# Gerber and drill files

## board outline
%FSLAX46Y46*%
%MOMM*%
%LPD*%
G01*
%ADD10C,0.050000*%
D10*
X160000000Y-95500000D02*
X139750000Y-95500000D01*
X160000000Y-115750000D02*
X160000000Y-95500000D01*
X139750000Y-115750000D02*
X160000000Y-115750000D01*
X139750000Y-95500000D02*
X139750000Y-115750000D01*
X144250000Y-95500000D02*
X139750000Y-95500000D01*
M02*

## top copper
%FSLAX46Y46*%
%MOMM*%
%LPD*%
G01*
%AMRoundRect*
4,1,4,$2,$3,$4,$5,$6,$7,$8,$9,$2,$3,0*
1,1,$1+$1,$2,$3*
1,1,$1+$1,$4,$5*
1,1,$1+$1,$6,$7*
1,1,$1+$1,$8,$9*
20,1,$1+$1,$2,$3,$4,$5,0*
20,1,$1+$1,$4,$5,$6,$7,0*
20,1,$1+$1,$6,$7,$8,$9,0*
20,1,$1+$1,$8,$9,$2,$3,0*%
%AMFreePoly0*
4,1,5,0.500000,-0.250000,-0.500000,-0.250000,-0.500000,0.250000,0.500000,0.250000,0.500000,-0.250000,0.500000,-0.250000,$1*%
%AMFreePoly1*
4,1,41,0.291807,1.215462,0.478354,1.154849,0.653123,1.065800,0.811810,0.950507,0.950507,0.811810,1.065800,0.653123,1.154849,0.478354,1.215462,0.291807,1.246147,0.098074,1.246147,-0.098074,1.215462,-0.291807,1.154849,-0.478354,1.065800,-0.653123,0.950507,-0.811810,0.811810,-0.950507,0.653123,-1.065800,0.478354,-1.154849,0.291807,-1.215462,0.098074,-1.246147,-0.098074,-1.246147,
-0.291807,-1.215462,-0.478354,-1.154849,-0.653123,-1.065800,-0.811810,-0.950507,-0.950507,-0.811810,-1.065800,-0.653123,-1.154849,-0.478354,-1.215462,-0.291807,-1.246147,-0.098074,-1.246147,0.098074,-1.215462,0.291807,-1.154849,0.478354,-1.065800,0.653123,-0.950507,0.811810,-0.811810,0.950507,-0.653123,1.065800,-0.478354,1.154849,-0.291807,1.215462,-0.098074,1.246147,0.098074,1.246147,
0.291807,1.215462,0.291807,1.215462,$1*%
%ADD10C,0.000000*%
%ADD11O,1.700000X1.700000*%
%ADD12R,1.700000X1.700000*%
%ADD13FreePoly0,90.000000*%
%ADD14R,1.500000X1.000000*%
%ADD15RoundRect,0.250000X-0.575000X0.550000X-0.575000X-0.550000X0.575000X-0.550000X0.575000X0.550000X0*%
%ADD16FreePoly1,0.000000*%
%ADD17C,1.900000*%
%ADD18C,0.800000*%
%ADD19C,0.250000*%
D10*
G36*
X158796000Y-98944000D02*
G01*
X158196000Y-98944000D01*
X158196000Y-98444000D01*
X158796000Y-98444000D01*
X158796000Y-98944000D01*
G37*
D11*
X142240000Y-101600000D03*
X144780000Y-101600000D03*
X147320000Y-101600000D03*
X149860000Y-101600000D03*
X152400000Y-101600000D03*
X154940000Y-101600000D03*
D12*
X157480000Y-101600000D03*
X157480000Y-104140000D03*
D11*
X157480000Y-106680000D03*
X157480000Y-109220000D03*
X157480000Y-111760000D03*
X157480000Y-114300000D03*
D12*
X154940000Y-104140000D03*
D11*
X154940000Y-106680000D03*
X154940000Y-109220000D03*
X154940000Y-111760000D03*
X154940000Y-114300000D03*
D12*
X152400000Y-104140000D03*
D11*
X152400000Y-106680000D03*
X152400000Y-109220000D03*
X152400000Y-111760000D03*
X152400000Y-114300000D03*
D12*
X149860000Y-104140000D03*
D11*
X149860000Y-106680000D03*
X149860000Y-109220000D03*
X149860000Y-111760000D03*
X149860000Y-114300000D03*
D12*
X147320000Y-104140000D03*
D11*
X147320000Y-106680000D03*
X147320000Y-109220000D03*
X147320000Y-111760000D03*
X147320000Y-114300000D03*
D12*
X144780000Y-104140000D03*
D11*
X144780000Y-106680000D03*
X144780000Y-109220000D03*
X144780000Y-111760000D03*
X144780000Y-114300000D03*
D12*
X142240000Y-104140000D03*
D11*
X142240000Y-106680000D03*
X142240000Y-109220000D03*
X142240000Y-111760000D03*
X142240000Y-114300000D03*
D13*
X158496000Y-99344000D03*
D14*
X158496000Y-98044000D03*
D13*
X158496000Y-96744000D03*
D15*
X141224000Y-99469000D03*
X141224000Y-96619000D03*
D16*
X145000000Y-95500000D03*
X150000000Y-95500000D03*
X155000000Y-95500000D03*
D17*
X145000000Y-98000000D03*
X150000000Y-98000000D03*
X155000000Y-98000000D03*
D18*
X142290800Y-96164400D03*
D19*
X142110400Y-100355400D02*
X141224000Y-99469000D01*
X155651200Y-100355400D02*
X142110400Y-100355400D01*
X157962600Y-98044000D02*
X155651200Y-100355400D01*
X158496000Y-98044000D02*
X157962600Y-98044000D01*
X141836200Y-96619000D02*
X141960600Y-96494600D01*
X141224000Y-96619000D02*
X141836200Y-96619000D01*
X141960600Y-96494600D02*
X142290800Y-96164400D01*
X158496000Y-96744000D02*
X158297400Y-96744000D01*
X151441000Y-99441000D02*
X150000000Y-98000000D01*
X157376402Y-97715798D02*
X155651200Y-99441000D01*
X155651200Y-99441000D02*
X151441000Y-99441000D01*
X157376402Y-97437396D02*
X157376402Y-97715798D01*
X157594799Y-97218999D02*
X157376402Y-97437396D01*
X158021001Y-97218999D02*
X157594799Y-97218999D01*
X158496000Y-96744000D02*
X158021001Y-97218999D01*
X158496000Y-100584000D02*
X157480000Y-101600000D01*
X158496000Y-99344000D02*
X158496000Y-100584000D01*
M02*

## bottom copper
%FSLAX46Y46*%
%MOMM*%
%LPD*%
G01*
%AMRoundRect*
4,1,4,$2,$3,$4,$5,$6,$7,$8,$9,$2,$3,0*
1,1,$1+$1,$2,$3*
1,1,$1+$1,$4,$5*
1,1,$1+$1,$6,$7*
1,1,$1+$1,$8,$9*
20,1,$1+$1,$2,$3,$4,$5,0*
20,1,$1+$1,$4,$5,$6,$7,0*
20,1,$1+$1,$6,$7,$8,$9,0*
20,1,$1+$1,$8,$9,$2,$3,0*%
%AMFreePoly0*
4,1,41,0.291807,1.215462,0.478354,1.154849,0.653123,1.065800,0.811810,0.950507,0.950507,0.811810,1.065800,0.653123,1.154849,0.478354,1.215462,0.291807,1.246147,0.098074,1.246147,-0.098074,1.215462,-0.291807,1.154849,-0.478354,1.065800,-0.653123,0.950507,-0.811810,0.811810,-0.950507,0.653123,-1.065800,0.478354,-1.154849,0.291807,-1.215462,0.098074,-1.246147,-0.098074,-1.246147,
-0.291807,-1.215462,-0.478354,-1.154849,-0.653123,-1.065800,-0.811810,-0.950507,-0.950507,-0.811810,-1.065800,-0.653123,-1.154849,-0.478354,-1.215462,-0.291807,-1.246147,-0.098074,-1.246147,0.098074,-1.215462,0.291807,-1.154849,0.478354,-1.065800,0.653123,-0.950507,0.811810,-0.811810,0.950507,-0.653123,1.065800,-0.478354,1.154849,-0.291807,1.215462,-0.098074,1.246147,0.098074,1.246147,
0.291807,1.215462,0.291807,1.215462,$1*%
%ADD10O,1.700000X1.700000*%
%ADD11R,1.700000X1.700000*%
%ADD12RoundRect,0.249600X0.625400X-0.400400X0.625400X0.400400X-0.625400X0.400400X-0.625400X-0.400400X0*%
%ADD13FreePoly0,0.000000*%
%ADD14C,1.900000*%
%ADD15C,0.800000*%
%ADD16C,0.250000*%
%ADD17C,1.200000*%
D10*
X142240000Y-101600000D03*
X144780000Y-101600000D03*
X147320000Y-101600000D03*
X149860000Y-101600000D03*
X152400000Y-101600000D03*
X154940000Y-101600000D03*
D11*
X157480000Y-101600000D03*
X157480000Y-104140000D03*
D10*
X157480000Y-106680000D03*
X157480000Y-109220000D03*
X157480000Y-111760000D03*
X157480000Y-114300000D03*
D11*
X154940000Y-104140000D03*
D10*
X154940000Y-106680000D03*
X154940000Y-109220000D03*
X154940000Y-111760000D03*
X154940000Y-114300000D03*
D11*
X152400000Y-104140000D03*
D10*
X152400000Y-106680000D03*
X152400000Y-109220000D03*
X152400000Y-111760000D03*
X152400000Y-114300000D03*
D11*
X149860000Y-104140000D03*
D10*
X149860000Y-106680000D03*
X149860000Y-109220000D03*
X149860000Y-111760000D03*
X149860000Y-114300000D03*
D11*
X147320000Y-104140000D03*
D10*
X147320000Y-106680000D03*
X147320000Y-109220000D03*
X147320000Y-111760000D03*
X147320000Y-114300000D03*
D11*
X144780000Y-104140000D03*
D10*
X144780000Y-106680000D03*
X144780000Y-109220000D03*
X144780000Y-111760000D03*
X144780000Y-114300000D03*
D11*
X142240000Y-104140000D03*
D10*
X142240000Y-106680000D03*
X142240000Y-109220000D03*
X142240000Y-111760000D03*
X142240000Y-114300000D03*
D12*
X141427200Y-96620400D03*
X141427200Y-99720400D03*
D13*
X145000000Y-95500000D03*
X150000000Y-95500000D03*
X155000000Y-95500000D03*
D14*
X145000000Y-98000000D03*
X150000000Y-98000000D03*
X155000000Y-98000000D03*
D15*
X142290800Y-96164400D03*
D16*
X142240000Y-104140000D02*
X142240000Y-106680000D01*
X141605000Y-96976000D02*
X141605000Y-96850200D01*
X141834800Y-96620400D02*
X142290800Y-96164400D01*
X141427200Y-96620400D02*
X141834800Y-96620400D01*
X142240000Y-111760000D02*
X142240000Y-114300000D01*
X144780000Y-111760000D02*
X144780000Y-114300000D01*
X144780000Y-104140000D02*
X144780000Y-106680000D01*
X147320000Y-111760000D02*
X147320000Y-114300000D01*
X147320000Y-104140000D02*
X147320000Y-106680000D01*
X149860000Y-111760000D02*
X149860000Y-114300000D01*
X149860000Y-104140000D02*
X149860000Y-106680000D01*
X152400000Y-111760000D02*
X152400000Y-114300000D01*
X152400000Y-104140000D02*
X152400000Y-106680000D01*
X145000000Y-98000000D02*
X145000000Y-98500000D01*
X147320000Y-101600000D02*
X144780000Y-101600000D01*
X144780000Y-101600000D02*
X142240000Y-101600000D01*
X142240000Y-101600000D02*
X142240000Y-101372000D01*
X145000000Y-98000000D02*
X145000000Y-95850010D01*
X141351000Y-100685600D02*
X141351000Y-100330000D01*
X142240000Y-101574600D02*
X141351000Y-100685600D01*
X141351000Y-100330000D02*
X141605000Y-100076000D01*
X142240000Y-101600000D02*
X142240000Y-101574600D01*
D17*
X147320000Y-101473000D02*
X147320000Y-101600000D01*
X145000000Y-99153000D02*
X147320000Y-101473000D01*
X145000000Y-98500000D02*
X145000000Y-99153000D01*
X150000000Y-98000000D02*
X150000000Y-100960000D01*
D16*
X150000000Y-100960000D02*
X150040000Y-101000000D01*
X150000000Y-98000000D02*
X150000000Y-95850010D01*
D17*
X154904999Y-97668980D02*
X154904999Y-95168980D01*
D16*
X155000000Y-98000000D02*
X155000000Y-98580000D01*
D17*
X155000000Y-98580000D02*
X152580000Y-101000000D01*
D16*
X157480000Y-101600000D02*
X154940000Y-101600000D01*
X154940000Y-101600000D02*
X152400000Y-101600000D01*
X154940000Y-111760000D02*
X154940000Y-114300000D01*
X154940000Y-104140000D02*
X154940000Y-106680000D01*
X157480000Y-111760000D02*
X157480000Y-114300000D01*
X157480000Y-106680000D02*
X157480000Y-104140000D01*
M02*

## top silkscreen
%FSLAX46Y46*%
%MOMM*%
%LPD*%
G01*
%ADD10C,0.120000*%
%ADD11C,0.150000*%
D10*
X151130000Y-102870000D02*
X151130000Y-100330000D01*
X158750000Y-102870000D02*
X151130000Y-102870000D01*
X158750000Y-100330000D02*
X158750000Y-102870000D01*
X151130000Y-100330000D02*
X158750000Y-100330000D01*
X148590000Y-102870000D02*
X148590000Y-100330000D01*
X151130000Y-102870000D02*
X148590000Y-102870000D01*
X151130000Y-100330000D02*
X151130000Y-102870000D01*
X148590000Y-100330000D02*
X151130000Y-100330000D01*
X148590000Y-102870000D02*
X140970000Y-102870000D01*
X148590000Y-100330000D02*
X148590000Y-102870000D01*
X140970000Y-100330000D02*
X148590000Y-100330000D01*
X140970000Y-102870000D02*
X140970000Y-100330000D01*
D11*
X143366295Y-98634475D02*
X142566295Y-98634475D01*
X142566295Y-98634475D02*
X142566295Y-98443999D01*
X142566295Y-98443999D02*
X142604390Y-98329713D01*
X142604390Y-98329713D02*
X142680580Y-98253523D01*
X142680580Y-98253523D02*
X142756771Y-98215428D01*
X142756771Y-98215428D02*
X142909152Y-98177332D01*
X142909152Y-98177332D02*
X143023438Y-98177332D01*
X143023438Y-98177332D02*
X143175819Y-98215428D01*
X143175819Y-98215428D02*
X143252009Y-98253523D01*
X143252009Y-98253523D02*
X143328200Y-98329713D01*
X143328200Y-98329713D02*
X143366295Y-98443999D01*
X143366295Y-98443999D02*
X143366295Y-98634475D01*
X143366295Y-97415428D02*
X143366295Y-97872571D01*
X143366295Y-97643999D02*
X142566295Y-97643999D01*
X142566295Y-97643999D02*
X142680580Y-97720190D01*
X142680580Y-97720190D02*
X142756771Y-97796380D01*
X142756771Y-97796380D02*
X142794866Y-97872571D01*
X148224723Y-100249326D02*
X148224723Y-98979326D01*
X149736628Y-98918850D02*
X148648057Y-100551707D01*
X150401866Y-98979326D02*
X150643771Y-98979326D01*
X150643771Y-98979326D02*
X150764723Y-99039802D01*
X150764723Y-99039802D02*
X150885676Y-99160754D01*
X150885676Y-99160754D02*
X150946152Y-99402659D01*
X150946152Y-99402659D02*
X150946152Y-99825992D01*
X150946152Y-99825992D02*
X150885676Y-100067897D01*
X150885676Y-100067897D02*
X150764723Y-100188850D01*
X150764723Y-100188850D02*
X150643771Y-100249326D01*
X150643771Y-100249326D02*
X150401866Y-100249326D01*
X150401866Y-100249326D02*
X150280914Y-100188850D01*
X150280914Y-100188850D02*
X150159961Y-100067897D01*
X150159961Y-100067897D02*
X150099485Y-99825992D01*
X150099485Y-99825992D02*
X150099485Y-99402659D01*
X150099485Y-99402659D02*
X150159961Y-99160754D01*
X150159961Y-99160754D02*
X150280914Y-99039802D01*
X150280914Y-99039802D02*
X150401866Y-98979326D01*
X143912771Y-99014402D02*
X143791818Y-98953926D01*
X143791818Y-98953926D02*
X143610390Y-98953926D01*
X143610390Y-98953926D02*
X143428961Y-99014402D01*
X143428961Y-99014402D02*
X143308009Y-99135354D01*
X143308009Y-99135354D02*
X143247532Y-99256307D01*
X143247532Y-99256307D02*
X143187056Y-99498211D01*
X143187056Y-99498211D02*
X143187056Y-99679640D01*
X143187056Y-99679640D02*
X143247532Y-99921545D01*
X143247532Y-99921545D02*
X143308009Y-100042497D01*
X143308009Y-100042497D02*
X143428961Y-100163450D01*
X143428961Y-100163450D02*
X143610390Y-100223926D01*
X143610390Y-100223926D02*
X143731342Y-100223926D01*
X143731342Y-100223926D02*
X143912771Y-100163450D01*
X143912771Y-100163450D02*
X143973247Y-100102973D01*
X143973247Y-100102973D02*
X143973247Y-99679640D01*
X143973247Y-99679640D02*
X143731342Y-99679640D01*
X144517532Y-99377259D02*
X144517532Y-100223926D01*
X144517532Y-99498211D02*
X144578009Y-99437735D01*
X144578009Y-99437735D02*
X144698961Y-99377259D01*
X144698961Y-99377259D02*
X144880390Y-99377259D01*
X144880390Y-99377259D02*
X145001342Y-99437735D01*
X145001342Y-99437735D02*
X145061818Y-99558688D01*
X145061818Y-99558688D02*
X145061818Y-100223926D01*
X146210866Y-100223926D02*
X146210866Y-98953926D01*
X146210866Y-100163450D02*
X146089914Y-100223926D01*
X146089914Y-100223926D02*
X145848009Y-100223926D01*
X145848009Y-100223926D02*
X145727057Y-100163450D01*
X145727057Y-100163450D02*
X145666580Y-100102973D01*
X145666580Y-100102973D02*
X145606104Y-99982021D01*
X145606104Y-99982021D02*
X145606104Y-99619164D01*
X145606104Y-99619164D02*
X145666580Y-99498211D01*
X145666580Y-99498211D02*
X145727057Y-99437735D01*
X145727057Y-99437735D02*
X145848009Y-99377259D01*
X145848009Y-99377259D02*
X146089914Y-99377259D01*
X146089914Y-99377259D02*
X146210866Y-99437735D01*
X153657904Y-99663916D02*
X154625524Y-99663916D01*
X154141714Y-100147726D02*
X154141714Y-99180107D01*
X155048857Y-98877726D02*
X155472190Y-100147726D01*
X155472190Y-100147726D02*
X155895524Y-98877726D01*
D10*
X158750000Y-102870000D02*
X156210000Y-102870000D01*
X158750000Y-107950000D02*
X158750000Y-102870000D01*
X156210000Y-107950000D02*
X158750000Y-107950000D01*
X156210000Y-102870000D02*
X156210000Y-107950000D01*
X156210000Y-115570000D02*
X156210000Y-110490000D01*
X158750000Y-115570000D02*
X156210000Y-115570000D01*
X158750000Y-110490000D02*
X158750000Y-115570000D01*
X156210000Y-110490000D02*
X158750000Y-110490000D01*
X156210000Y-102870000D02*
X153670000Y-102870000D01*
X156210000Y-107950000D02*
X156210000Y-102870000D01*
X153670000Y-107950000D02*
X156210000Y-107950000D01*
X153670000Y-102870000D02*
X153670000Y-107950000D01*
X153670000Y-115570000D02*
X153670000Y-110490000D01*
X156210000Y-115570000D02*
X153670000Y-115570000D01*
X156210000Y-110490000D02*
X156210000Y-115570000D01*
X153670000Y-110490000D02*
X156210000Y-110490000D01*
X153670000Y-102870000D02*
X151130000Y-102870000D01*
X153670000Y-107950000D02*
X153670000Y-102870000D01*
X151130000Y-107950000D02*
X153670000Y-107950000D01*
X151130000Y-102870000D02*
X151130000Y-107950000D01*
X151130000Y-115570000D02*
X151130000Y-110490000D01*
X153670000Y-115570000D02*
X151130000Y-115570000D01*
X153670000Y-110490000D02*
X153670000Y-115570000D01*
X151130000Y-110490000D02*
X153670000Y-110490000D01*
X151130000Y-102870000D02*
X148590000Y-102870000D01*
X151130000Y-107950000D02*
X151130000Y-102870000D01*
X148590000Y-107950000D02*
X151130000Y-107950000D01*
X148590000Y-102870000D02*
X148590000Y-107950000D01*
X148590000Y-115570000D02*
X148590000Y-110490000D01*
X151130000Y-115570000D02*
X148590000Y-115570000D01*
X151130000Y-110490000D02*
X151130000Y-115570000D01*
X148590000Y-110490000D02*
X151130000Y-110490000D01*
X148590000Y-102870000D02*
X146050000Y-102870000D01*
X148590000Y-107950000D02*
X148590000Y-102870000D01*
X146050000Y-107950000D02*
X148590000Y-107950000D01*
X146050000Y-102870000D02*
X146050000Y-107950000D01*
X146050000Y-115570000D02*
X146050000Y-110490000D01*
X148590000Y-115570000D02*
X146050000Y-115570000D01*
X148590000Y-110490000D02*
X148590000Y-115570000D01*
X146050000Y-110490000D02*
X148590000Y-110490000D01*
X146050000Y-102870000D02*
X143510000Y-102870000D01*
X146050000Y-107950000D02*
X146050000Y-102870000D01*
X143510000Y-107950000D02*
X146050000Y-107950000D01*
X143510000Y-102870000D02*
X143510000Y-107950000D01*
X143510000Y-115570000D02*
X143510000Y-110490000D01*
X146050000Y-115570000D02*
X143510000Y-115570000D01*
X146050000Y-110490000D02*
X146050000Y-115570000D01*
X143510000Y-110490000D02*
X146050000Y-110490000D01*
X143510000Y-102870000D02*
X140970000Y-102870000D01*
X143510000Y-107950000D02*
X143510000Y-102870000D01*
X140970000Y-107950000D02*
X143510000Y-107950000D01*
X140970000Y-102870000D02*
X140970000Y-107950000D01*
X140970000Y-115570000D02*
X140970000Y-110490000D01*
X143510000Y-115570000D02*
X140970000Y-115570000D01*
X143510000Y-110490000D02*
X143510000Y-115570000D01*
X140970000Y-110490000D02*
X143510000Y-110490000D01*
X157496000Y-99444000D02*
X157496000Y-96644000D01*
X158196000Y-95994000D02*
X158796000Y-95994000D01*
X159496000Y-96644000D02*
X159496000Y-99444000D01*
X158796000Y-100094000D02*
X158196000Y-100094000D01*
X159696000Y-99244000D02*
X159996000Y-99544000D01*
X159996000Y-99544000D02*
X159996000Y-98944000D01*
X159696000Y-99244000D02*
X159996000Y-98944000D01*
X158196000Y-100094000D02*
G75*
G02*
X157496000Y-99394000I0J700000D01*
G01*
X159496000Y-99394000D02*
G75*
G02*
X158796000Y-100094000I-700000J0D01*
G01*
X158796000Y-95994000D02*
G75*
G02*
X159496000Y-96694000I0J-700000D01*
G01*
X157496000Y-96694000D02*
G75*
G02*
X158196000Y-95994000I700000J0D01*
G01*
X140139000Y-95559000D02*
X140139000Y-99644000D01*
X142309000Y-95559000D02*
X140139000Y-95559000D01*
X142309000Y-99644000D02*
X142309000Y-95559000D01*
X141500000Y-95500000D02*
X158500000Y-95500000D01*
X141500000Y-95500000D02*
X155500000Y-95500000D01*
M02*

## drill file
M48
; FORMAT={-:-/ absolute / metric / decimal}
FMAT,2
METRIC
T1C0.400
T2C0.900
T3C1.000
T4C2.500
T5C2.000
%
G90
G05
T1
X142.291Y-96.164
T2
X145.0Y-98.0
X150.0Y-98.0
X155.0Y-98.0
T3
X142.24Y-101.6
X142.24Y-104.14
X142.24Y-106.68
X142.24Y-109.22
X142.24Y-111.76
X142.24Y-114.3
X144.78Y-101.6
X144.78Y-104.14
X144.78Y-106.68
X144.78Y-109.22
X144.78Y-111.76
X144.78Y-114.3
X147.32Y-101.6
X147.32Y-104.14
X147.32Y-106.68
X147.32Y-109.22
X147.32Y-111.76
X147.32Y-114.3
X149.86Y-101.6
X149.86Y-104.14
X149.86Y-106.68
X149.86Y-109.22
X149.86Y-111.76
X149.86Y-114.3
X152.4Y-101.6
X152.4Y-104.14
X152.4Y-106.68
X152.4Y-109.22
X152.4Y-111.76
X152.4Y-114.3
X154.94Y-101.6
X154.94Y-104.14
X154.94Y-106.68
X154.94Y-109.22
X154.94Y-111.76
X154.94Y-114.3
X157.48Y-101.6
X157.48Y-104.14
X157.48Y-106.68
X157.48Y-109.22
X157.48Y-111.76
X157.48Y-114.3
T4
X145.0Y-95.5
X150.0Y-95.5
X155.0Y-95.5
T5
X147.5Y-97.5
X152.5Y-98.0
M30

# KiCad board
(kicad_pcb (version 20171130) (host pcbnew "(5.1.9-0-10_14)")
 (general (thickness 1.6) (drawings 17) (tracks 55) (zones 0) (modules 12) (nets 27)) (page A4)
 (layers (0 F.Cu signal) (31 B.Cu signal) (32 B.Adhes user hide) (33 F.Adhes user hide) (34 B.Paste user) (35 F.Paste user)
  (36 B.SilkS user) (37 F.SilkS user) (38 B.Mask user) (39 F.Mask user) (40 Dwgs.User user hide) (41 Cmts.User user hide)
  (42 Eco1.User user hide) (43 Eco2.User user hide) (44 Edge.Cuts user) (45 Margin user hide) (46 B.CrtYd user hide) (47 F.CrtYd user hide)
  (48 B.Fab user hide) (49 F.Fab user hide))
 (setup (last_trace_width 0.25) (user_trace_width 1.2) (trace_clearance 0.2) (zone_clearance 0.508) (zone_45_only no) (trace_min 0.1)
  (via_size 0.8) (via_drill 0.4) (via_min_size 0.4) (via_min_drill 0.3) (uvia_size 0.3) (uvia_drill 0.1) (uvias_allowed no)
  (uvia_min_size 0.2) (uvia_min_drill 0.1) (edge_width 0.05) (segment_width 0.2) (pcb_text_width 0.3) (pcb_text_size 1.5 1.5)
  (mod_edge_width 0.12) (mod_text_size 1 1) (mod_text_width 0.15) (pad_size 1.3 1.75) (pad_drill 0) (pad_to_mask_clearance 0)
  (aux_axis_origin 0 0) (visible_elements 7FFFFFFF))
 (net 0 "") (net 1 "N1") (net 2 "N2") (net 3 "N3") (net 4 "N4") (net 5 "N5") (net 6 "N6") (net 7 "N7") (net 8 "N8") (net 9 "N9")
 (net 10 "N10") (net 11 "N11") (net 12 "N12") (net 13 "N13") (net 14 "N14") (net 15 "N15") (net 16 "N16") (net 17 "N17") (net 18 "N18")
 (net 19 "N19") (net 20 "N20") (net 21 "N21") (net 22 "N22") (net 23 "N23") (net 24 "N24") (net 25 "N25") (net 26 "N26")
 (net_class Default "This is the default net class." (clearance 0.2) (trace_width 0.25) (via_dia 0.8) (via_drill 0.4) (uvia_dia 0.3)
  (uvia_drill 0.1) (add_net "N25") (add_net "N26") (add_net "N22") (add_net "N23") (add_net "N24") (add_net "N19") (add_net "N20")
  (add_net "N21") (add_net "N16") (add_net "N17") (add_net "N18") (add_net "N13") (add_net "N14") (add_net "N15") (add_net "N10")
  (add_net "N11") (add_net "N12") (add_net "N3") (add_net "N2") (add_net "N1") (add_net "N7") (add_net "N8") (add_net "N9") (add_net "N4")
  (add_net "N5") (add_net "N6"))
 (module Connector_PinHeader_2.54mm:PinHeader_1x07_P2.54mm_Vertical (layer F.Cu) (at 157.48 101.6 270)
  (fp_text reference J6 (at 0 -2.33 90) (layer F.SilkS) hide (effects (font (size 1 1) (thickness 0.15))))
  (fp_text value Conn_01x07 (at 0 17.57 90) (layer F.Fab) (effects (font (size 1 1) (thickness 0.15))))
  (pad 7 thru_hole oval (at 0 15.24 270) (size 1.7 1.7) (drill 1) (layers *.Cu *.Mask) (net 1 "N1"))
  (pad 6 thru_hole oval (at 0 12.7 270) (size 1.7 1.7) (drill 1) (layers *.Cu *.Mask) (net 1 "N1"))
  (pad 5 thru_hole oval (at 0 10.16 270) (size 1.7 1.7) (drill 1) (layers *.Cu *.Mask) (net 1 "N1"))
  (pad 4 thru_hole oval (at 0 7.62 270) (size 1.7 1.7) (drill 1) (layers *.Cu *.Mask) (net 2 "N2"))
  (pad 3 thru_hole oval (at 0 5.08 270) (size 1.7 1.7) (drill 1) (layers *.Cu *.Mask) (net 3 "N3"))
  (pad 2 thru_hole oval (at 0 2.54 270) (size 1.7 1.7) (drill 1) (layers *.Cu *.Mask) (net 3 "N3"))
  (pad 1 thru_hole rect (at 0 0 270) (size 1.7 1.7) (drill 1) (layers *.Cu *.Mask) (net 3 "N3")))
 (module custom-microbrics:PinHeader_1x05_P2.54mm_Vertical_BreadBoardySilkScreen (layer F.Cu) (at 157.48 104.14)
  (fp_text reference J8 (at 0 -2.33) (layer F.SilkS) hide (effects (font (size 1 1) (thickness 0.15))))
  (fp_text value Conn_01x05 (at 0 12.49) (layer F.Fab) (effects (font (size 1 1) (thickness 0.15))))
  (fp_line (start 1.27 -1.27) (end -1.27 -1.27) (layer F.SilkS) (width 0.12))
  (fp_line (start 1.27 3.81) (end 1.27 -1.27) (layer F.SilkS) (width 0.12))
  (fp_line (start -1.27 3.81) (end 1.27 3.81) (layer F.SilkS) (width 0.12))
  (fp_line (start -1.27 -1.27) (end -1.27 3.81) (layer F.SilkS) (width 0.12))
  (fp_line (start -1.27 11.43) (end -1.27 6.35) (layer F.SilkS) (width 0.12))
  (fp_line (start 1.27 11.43) (end -1.27 11.43) (layer F.SilkS) (width 0.12))
  (fp_line (start 1.27 6.35) (end 1.27 11.43) (layer F.SilkS) (width 0.12))
  (fp_line (start -1.27 6.35) (end 1.27 6.35) (layer F.SilkS) (width 0.12))
  (pad 1 thru_hole rect (at 0 0) (size 1.7 1.7) (drill 1) (layers *.Cu *.Mask) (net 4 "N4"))
  (pad 2 thru_hole oval (at 0 2.54) (size 1.7 1.7) (drill 1) (layers *.Cu *.Mask) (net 4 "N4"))
  (pad 3 thru_hole oval (at 0 5.08) (size 1.7 1.7) (drill 1) (layers *.Cu *.Mask) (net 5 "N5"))
  (pad 4 thru_hole oval (at 0 7.62) (size 1.7 1.7) (drill 1) (layers *.Cu *.Mask) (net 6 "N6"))
  (pad 5 thru_hole oval (at 0 10.16) (size 1.7 1.7) (drill 1) (layers *.Cu *.Mask) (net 6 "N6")))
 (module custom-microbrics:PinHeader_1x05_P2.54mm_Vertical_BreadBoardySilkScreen (layer F.Cu) (at 154.94 104.14)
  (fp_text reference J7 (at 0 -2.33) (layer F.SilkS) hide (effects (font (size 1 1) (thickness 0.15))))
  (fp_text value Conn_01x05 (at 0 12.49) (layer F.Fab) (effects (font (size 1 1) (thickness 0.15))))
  (fp_line (start 1.27 -1.27) (end -1.27 -1.27) (layer F.SilkS) (width 0.12))
  (fp_line (start 1.27 3.81) (end 1.27 -1.27) (layer F.SilkS) (width 0.12))
  (fp_line (start -1.27 3.81) (end 1.27 3.81) (layer F.SilkS) (width 0.12))
  (fp_line (start -1.27 -1.27) (end -1.27 3.81) (layer F.SilkS) (width 0.12))
  (fp_line (start -1.27 11.43) (end -1.27 6.35) (layer F.SilkS) (width 0.12))
  (fp_line (start 1.27 11.43) (end -1.27 11.43) (layer F.SilkS) (width 0.12))
  (fp_line (start 1.27 6.35) (end 1.27 11.43) (layer F.SilkS) (width 0.12))
  (fp_line (start -1.27 6.35) (end 1.27 6.35) (layer F.SilkS) (width 0.12))
  (pad 1 thru_hole rect (at 0 0) (size 1.7 1.7) (drill 1) (layers *.Cu *.Mask) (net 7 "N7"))
  (pad 2 thru_hole oval (at 0 2.54) (size 1.7 1.7) (drill 1) (layers *.Cu *.Mask) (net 7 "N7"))
  (pad 3 thru_hole oval (at 0 5.08) (size 1.7 1.7) (drill 1) (layers *.Cu *.Mask) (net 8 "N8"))
  (pad 4 thru_hole oval (at 0 7.62) (size 1.7 1.7) (drill 1) (layers *.Cu *.Mask) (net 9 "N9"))
  (pad 5 thru_hole oval (at 0 10.16) (size 1.7 1.7) (drill 1) (layers *.Cu *.Mask) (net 9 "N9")))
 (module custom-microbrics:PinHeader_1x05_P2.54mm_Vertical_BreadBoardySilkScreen (layer F.Cu) (at 152.4 104.14)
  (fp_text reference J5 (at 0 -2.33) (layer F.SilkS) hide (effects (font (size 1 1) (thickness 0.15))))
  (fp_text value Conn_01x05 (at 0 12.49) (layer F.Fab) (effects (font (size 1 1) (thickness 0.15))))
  (fp_line (start 1.27 -1.27) (end -1.27 -1.27) (layer F.SilkS) (width 0.12))
  (fp_line (start 1.27 3.81) (end 1.27 -1.27) (layer F.SilkS) (width 0.12))
  (fp_line (start -1.27 3.81) (end 1.27 3.81) (layer F.SilkS) (width 0.12))
  (fp_line (start -1.27 -1.27) (end -1.27 3.81) (layer F.SilkS) (width 0.12))
  (fp_line (start -1.27 11.43) (end -1.27 6.35) (layer F.SilkS) (width 0.12))
  (fp_line (start 1.27 11.43) (end -1.27 11.43) (layer F.SilkS) (width 0.12))
  (fp_line (start 1.27 6.35) (end 1.27 11.43) (layer F.SilkS) (width 0.12))
  (fp_line (start -1.27 6.35) (end 1.27 6.35) (layer F.SilkS) (width 0.12))
  (pad 1 thru_hole rect (at 0 0) (size 1.7 1.7) (drill 1) (layers *.Cu *.Mask) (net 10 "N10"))
  (pad 2 thru_hole oval (at 0 2.54) (size 1.7 1.7) (drill 1) (layers *.Cu *.Mask) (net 10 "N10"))
  (pad 3 thru_hole oval (at 0 5.08) (size 1.7 1.7) (drill 1) (layers *.Cu *.Mask) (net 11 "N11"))
  (pad 4 thru_hole oval (at 0 7.62) (size 1.7 1.7) (drill 1) (layers *.Cu *.Mask) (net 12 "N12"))
  (pad 5 thru_hole oval (at 0 10.16) (size 1.7 1.7) (drill 1) (layers *.Cu *.Mask) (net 12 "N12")))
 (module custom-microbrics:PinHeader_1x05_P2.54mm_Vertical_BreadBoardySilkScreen (layer F.Cu) (at 149.86 104.14)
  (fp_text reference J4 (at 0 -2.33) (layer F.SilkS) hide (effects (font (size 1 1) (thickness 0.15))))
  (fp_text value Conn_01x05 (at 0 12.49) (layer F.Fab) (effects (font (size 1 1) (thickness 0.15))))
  (fp_line (start 1.27 -1.27) (end -1.27 -1.27) (layer F.SilkS) (width 0.12))
  (fp_line (start 1.27 3.81) (end 1.27 -1.27) (layer F.SilkS) (width 0.12))
  (fp_line (start -1.27 3.81) (end 1.27 3.81) (layer F.SilkS) (width 0.12))
  (fp_line (start -1.27 -1.27) (end -1.27 3.81) (layer F.SilkS) (width 0.12))
  (fp_line (start -1.27 11.43) (end -1.27 6.35) (layer F.SilkS) (width 0.12))
  (fp_line (start 1.27 11.43) (end -1.27 11.43) (layer F.SilkS) (width 0.12))
  (fp_line (start 1.27 6.35) (end 1.27 11.43) (layer F.SilkS) (width 0.12))
  (fp_line (start -1.27 6.35) (end 1.27 6.35) (layer F.SilkS) (width 0.12))
  (pad 1 thru_hole rect (at 0 0) (size 1.7 1.7) (drill 1) (layers *.Cu *.Mask) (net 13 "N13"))
  (pad 2 thru_hole oval (at 0 2.54) (size 1.7 1.7) (drill 1) (layers *.Cu *.Mask) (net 13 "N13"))
  (pad 3 thru_hole oval (at 0 5.08) (size 1.7 1.7) (drill 1) (layers *.Cu *.Mask) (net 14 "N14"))
  (pad 4 thru_hole oval (at 0 7.62) (size 1.7 1.7) (drill 1) (layers *.Cu *.Mask) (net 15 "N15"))
  (pad 5 thru_hole oval (at 0 10.16) (size 1.7 1.7) (drill 1) (layers *.Cu *.Mask) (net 15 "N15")))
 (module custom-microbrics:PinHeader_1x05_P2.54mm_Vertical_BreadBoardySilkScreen (layer F.Cu) (at 147.32 104.14)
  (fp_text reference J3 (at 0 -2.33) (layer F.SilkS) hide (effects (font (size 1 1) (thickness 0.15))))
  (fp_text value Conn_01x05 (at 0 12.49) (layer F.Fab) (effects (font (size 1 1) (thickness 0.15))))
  (fp_line (start 1.27 -1.27) (end -1.27 -1.27) (layer F.SilkS) (width 0.12))
  (fp_line (start 1.27 3.81) (end 1.27 -1.27) (layer F.SilkS) (width 0.12))
  (fp_line (start -1.27 3.81) (end 1.27 3.81) (layer F.SilkS) (width 0.12))
  (fp_line (start -1.27 -1.27) (end -1.27 3.81) (layer F.SilkS) (width 0.12))
  (fp_line (start -1.27 11.43) (end -1.27 6.35) (layer F.SilkS) (width 0.12))
  (fp_line (start 1.27 11.43) (end -1.27 11.43) (layer F.SilkS) (width 0.12))
  (fp_line (start 1.27 6.35) (end 1.27 11.43) (layer F.SilkS) (width 0.12))
  (fp_line (start -1.27 6.35) (end 1.27 6.35) (layer F.SilkS) (width 0.12))
  (pad 1 thru_hole rect (at 0 0) (size 1.7 1.7) (drill 1) (layers *.Cu *.Mask) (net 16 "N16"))
  (pad 2 thru_hole oval (at 0 2.54) (size 1.7 1.7) (drill 1) (layers *.Cu *.Mask) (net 16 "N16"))
  (pad 3 thru_hole oval (at 0 5.08) (size 1.7 1.7) (drill 1) (layers *.Cu *.Mask) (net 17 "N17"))
  (pad 4 thru_hole oval (at 0 7.62) (size 1.7 1.7) (drill 1) (layers *.Cu *.Mask) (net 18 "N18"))
  (pad 5 thru_hole oval (at 0 10.16) (size 1.7 1.7) (drill 1) (layers *.Cu *.Mask) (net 18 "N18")))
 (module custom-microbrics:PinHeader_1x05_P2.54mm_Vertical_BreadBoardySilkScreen (layer F.Cu) (at 144.78 104.14)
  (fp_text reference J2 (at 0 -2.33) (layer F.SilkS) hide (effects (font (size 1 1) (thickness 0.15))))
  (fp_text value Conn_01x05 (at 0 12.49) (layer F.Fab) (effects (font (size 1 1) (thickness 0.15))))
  (fp_line (start 1.27 -1.27) (end -1.27 -1.27) (layer F.SilkS) (width 0.12))
  (fp_line (start 1.27 3.81) (end 1.27 -1.27) (layer F.SilkS) (width 0.12))
  (fp_line (start -1.27 3.81) (end 1.27 3.81) (layer F.SilkS) (width 0.12))
  (fp_line (start -1.27 -1.27) (end -1.27 3.81) (layer F.SilkS) (width 0.12))
  (fp_line (start -1.27 11.43) (end -1.27 6.35) (layer F.SilkS) (width 0.12))
  (fp_line (start 1.27 11.43) (end -1.27 11.43) (layer F.SilkS) (width 0.12))
  (fp_line (start 1.27 6.35) (end 1.27 11.43) (layer F.SilkS) (width 0.12))
  (fp_line (start -1.27 6.35) (end 1.27 6.35) (layer F.SilkS) (width 0.12))
  (pad 1 thru_hole rect (at 0 0) (size 1.7 1.7) (drill 1) (layers *.Cu *.Mask) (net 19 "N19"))
  (pad 2 thru_hole oval (at 0 2.54) (size 1.7 1.7) (drill 1) (layers *.Cu *.Mask) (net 19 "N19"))
  (pad 3 thru_hole oval (at 0 5.08) (size 1.7 1.7) (drill 1) (layers *.Cu *.Mask) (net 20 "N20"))
  (pad 4 thru_hole oval (at 0 7.62) (size 1.7 1.7) (drill 1) (layers *.Cu *.Mask) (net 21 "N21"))
  (pad 5 thru_hole oval (at 0 10.16) (size 1.7 1.7) (drill 1) (layers *.Cu *.Mask) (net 21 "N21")))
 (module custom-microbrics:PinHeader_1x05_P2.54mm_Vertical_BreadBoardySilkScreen (layer F.Cu) (at 142.24 104.14)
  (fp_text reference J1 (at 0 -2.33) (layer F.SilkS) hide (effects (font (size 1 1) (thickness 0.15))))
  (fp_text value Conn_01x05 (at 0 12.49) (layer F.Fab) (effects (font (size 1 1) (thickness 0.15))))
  (fp_line (start 1.27 -1.27) (end -1.27 -1.27) (layer F.SilkS) (width 0.12))
  (fp_line (start 1.27 3.81) (end 1.27 -1.27) (layer F.SilkS) (width 0.12))
  (fp_line (start -1.27 3.81) (end 1.27 3.81) (layer F.SilkS) (width 0.12))
  (fp_line (start -1.27 -1.27) (end -1.27 3.81) (layer F.SilkS) (width 0.12))
  (fp_line (start -1.27 11.43) (end -1.27 6.35) (layer F.SilkS) (width 0.12))
  (fp_line (start 1.27 11.43) (end -1.27 11.43) (layer F.SilkS) (width 0.12))
  (fp_line (start 1.27 6.35) (end 1.27 11.43) (layer F.SilkS) (width 0.12))
  (fp_line (start -1.27 6.35) (end 1.27 6.35) (layer F.SilkS) (width 0.12))
  (pad 1 thru_hole rect (at 0 0) (size 1.7 1.7) (drill 1) (layers *.Cu *.Mask) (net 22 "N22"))
  (pad 2 thru_hole oval (at 0 2.54) (size 1.7 1.7) (drill 1) (layers *.Cu *.Mask) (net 22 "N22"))
  (pad 3 thru_hole oval (at 0 5.08) (size 1.7 1.7) (drill 1) (layers *.Cu *.Mask) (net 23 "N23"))
  (pad 4 thru_hole oval (at 0 7.62) (size 1.7 1.7) (drill 1) (layers *.Cu *.Mask) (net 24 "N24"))
  (pad 5 thru_hole oval (at 0 10.16) (size 1.7 1.7) (drill 1) (layers *.Cu *.Mask) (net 24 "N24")))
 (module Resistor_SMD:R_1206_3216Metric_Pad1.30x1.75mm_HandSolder (layer B.Cu) (at 141.4272 98.1704 90)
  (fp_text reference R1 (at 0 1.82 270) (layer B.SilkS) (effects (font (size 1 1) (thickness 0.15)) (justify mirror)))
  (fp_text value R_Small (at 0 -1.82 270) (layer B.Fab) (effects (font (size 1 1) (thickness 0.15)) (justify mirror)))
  (pad 2 smd roundrect (at 1.55 0 90) (size 1.3 1.75) (layers B.Cu B.Paste B.Mask) (roundrect_rratio 0.192) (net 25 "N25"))
  (pad 1 smd roundrect (at -1.55 0 90) (size 1.3 1.75) (layers B.Cu B.Paste B.Mask) (roundrect_rratio 0.192) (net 1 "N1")))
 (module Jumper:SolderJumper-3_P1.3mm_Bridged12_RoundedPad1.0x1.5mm (layer F.Cu) (at 158.496 98.044 90)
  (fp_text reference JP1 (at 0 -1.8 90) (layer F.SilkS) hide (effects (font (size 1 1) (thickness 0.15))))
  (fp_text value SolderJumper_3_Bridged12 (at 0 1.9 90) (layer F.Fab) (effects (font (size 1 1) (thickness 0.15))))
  (fp_poly (pts (xy -0.9 -0.3) (xy -0.4 -0.3) (xy -0.4 0.3) (xy -0.9 0.3)) (layer F.Cu) (width 0))
  (fp_line (start -1.4 -1) (end 1.4 -1) (layer F.SilkS) (width 0.12))
  (fp_line (start 2.05 -0.3) (end 2.05 0.3) (layer F.SilkS) (width 0.12))
  (fp_line (start 1.4 1) (end -1.4 1) (layer F.SilkS) (width 0.12))
  (fp_line (start -2.05 0.3) (end -2.05 -0.3) (layer F.SilkS) (width 0.12))
  (fp_line (start -1.2 1.2) (end -1.5 1.5) (layer F.SilkS) (width 0.12))
  (fp_line (start -1.5 1.5) (end -0.9 1.5) (layer F.SilkS) (width 0.12))
  (fp_line (start -1.2 1.2) (end -0.9 1.5) (layer F.SilkS) (width 0.12))
  (fp_arc (start -1.35 -0.3) (end -1.35 -1) (angle -90) (layer F.SilkS) (width 0.12))
  (fp_arc (start -1.35 0.3) (end -2.05 0.3) (angle -90) (layer F.SilkS) (width 0.12))
  (fp_arc (start 1.35 0.3) (end 1.35 1) (angle -90) (layer F.SilkS) (width 0.12))
  (fp_arc (start 1.35 -0.3) (end 2.05 -0.3) (angle -90) (layer F.SilkS) (width 0.12))
  (pad 1 smd custom (at -1.3 0 90) (size 1 0.5) (layers F.Cu F.Mask) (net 3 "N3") (zone_connect 2)
   (options (clearance outline) (anchor rect)) (primitives))
  (pad 2 smd rect (at 0 0 90) (size 1 1.5) (layers F.Cu F.Mask) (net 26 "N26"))
  (pad 3 smd custom (at 1.3 0 90) (size 1 0.5) (layers F.Cu F.Mask) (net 2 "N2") (zone_connect 2)
   (options (clearance outline) (anchor rect)) (primitives)))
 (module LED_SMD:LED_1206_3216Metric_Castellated (layer F.Cu) (at 141.224 98.044 270)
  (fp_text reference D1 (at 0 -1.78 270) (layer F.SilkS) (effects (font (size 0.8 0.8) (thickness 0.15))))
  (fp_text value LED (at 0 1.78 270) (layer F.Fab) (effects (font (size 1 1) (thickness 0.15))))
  (fp_line (start -2.485 1.085) (end 1.6 1.085) (layer F.SilkS) (width 0.12))
  (fp_line (start -2.485 -1.085) (end -2.485 1.085) (layer F.SilkS) (width 0.12))
  (fp_line (start 1.6 -1.085) (end -2.485 -1.085) (layer F.SilkS) (width 0.12))
  (pad 2 smd roundrect (at 1.425 0 270) (size 1.6 1.65) (layers F.Cu F.Paste F.Mask) (roundrect_rratio 0.15625) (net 26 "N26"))
  (pad 1 smd roundrect (at -1.425 0 270) (size 1.6 1.65) (layers F.Cu F.Paste F.Mask) (roundrect_rratio 0.15625) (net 25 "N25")))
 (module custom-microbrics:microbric (layer F.Cu) (at 141 101.5)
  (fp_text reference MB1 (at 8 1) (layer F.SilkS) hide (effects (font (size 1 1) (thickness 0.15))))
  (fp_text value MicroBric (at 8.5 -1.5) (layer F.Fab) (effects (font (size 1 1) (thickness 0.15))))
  (fp_line (start 0.5 -6) (end 17.5 -6) (layer F.SilkS) (width 0.12))
  (fp_line (start 0.5 -6) (end 14.5 -6) (layer F.SilkS) (width 0.12))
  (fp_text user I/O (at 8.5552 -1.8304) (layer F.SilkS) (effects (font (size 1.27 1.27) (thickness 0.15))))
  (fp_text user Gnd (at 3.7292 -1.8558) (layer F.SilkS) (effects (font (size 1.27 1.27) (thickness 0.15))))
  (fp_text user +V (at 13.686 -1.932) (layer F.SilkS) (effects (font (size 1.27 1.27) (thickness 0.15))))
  (pad 1 thru_hole custom (at 4 -6) (size 2.5 2.5) (drill 2.5) (layers *.Cu *.Mask) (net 1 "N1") (zone_connect 0)
   (options (clearance outline) (anchor circle)) (primitives))
  (pad 2 thru_hole custom (at 9 -6) (size 2.5 2.5) (drill 2.5) (layers *.Cu *.Mask) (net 2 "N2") (zone_connect 0)
   (options (clearance outline) (anchor circle)) (primitives))
  (pad 3 thru_hole custom (at 14 -6) (size 2.5 2.5) (drill 2.5) (layers *.Cu *.Mask) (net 3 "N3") (zone_connect 0)
   (options (clearance outline) (anchor circle)) (primitives))
  (pad 1 thru_hole circle (at 4 -3.5) (size 1.9 1.9) (drill 0.9) (layers *.Cu *.Mask) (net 1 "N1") (zone_connect 0))
  (pad 2 thru_hole circle (at 9 -3.5) (size 1.9 1.9) (drill 0.9) (layers *.Cu *.Mask) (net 2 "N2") (zone_connect 0))
  (pad 3 thru_hole circle (at 14 -3.5) (size 1.9 1.9) (drill 0.9) (layers *.Cu *.Mask) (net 3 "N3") (zone_connect 0))
  (pad "" np_thru_hole circle (at 6.5 -4) (size 2 2) (drill 2) (layers *.Cu *.Mask) (zone_connect 0))
  (pad "" np_thru_hole circle (at 11.5 -3.5) (size 2 2) (drill 2) (layers *.Cu *.Mask) (zone_connect 0)))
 (gr_line (start 151.13 102.87) (end 151.13 100.33) (angle 90) (layer F.SilkS) (width 0.12))
 (gr_line (start 158.75 102.87) (end 151.13 102.87) (angle 90) (layer F.SilkS) (width 0.12))
 (gr_line (start 158.75 100.33) (end 158.75 102.87) (angle 90) (layer F.SilkS) (width 0.12))
 (gr_line (start 151.13 100.33) (end 158.75 100.33) (angle 90) (layer F.SilkS) (width 0.12))
 (gr_line (start 148.59 102.87) (end 148.59 100.33) (angle 90) (layer F.SilkS) (width 0.12))
 (gr_line (start 151.13 102.87) (end 148.59 102.87) (angle 90) (layer F.SilkS) (width 0.12))
 (gr_line (start 151.13 100.33) (end 151.13 102.87) (angle 90) (layer F.SilkS) (width 0.12))
 (gr_line (start 148.59 100.33) (end 151.13 100.33) (angle 90) (layer F.SilkS) (width 0.12))
 (gr_line (start 148.59 102.87) (end 140.97 102.87) (angle 90) (layer F.SilkS) (width 0.12))
 (gr_line (start 148.59 100.33) (end 148.59 102.87) (angle 90) (layer F.SilkS) (width 0.12))
 (gr_line (start 140.97 100.33) (end 148.59 100.33) (angle 90) (layer F.SilkS) (width 0.12))
 (gr_line (start 140.97 102.87) (end 140.97 100.33) (angle 90) (layer F.SilkS) (width 0.12))
 (gr_line (start 160 95.5) (end 139.75 95.5) (layer Edge.Cuts) (width 0.05))
 (gr_line (start 160 115.75) (end 160 95.5) (layer Edge.Cuts) (width 0.05))
 (gr_line (start 139.75 115.75) (end 160 115.75) (layer Edge.Cuts) (width 0.05))
 (gr_line (start 139.75 95.5) (end 139.75 115.75) (layer Edge.Cuts) (width 0.05))
 (gr_line (start 144.25 95.5) (end 139.75 95.5) (layer Edge.Cuts) (width 0.05))
 (segment (start 142.24 104.14) (end 142.24 106.68) (width 0.25) (layer B.Cu) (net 22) (status C00000))
 (segment (start 142.1104 100.3554) (end 141.224 99.469) (width 0.25) (layer F.Cu) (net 26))
 (segment (start 155.6512 100.3554) (end 142.1104 100.3554) (width 0.25) (layer F.Cu) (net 26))
 (segment (start 157.9626 98.044) (end 155.6512 100.3554) (width 0.25) (layer F.Cu) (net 26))
 (segment (start 158.496 98.044) (end 157.9626 98.044) (width 0.25) (layer F.Cu) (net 26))
 (via (at 142.2908 96.1644) (size 0.8) (drill 0.4) (layers F.Cu B.Cu) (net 25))
 (segment (start 141.605 96.976) (end 141.605 96.8502) (width 0.25) (layer B.Cu) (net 25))
 (segment (start 141.8348 96.6204) (end 142.2908 96.1644) (width 0.25) (layer B.Cu) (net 25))
 (segment (start 141.4272 96.6204) (end 141.8348 96.6204) (width 0.25) (layer B.Cu) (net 25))
 (segment (start 141.8362 96.619) (end 141.9606 96.4946) (width 0.25) (layer F.Cu) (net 25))
 (segment (start 141.224 96.619) (end 141.8362 96.619) (width 0.25) (layer F.Cu) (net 25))
 (segment (start 141.9606 96.4946) (end 142.2908 96.1644) (width 0.25) (layer F.Cu) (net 25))
 (segment (start 142.24 111.76) (end 142.24 114.3) (width 0.25) (layer B.Cu) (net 24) (status C00000))
 (segment (start 144.78 111.76) (end 144.78 114.3) (width 0.25) (layer B.Cu) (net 21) (status C00000))
 (segment (start 144.78 104.14) (end 144.78 106.68) (width 0.25) (layer B.Cu) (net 19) (status C00000))
 (segment (start 147.32 111.76) (end 147.32 114.3) (width 0.25) (layer B.Cu) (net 18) (status C00000))
 (segment (start 147.32 104.14) (end 147.32 106.68) (width 0.25) (layer B.Cu) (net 16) (status C00000))
 (segment (start 149.86 111.76) (end 149.86 114.3) (width 0.25) (layer B.Cu) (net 15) (status C00000))
 (segment (start 149.86 104.14) (end 149.86 106.68) (width 0.25) (layer B.Cu) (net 13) (status C00000))
 (segment (start 152.4 111.76) (end 152.4 114.3) (width 0.25) (layer B.Cu) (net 12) (status C00000))
 (segment (start 152.4 104.14) (end 152.4 106.68) (width 0.25) (layer B.Cu) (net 10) (status C00000))
 (segment (start 145 98) (end 145 98.5) (width 0.25) (layer B.Cu) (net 1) (status C00000))
 (segment (start 147.32 101.6) (end 144.78 101.6) (width 0.25) (layer B.Cu) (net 1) (status C00000))
 (segment (start 144.78 101.6) (end 142.24 101.6) (width 0.25) (layer B.Cu) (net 1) (status C00000))
 (segment (start 142.24 101.6) (end 142.24 101.372) (width 0.25) (layer B.Cu) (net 1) (status C00000))
 (segment (start 145 98) (end 145 95.85001) (width 0.25) (layer B.Cu) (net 1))
 (segment (start 141.351 100.6856) (end 141.351 100.33) (width 0.25) (layer B.Cu) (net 1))
 (segment (start 142.24 101.5746) (end 141.351 100.6856) (width 0.25) (layer B.Cu) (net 1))
 (segment (start 141.351 100.33) (end 141.605 100.076) (width 0.25) (layer B.Cu) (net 1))
 (segment (start 142.24 101.6) (end 142.24 101.5746) (width 0.25) (layer B.Cu) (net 1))
 (segment (start 147.32 101.473) (end 147.32 101.6) (width 1.2) (layer B.Cu) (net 1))
 (segment (start 145 99.153) (end 147.32 101.473) (width 1.2) (layer B.Cu) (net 1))
 (segment (start 145 98.5) (end 145 99.153) (width 1.2) (layer B.Cu) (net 1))
 (segment (start 150 98) (end 150 100.96) (width 1.2) (layer B.Cu) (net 2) (status C00000))
 (segment (start 150 100.96) (end 150.04 101) (width 0.25) (layer B.Cu) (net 2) (status C00000))
 (segment (start 150 98) (end 150 95.85001) (width 0.25) (layer B.Cu) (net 2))
 (segment (start 158.496 96.744) (end 158.2974 96.744) (width 0.25) (layer F.Cu) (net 2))
 (segment (start 151.441 99.441) (end 150 98) (width 0.25) (layer F.Cu) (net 2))
 (segment (start 157.376402 97.715798) (end 155.6512 99.441) (width 0.25) (layer F.Cu) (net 2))
 (segment (start 155.6512 99.441) (end 151.441 99.441) (width 0.25) (layer F.Cu) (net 2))
 (segment (start 157.376402 97.437396) (end 157.376402 97.715798) (width 0.25) (layer F.Cu) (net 2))
 (segment (start 157.594799 97.218999) (end 157.376402 97.437396) (width 0.25) (layer F.Cu) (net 2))
 (segment (start 158.021001 97.218999) (end 157.594799 97.218999) (width 0.25) (layer F.Cu) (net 2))
 (segment (start 158.496 96.744) (end 158.021001 97.218999) (width 0.25) (layer F.Cu) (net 2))
 (segment (start 154.904999 97.66898) (end 154.904999 95.16898) (width 1.2) (layer B.Cu) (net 3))
 (segment (start 155 98) (end 155 98.58) (width 0.25) (layer B.Cu) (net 3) (status C00000))
 (segment (start 155 98.58) (end 152.58 101) (width 1.2) (layer B.Cu) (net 3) (status C00000))
 (segment (start 157.48 101.6) (end 154.94 101.6) (width 0.25) (layer B.Cu) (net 3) (status C00000))
 (segment (start 154.94 101.6) (end 152.4 101.6) (width 0.25) (layer B.Cu) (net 3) (status C00000))
 (segment (start 158.496 100.584) (end 157.48 101.6) (width 0.25) (layer F.Cu) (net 3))
 (segment (start 158.496 99.344) (end 158.496 100.584) (width 0.25) (layer F.Cu) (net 3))
 (segment (start 154.94 111.76) (end 154.94 114.3) (width 0.25) (layer B.Cu) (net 9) (status C00000))
 (segment (start 154.94 104.14) (end 154.94 106.68) (width 0.25) (layer B.Cu) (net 7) (status C00000))
 (segment (start 157.48 111.76) (end 157.48 114.3) (width 0.25) (layer B.Cu) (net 6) (status C00000))
 (segment (start 157.48 106.68) (end 157.48 104.14) (width 0.25) (layer B.Cu) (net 4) (status C00000)))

